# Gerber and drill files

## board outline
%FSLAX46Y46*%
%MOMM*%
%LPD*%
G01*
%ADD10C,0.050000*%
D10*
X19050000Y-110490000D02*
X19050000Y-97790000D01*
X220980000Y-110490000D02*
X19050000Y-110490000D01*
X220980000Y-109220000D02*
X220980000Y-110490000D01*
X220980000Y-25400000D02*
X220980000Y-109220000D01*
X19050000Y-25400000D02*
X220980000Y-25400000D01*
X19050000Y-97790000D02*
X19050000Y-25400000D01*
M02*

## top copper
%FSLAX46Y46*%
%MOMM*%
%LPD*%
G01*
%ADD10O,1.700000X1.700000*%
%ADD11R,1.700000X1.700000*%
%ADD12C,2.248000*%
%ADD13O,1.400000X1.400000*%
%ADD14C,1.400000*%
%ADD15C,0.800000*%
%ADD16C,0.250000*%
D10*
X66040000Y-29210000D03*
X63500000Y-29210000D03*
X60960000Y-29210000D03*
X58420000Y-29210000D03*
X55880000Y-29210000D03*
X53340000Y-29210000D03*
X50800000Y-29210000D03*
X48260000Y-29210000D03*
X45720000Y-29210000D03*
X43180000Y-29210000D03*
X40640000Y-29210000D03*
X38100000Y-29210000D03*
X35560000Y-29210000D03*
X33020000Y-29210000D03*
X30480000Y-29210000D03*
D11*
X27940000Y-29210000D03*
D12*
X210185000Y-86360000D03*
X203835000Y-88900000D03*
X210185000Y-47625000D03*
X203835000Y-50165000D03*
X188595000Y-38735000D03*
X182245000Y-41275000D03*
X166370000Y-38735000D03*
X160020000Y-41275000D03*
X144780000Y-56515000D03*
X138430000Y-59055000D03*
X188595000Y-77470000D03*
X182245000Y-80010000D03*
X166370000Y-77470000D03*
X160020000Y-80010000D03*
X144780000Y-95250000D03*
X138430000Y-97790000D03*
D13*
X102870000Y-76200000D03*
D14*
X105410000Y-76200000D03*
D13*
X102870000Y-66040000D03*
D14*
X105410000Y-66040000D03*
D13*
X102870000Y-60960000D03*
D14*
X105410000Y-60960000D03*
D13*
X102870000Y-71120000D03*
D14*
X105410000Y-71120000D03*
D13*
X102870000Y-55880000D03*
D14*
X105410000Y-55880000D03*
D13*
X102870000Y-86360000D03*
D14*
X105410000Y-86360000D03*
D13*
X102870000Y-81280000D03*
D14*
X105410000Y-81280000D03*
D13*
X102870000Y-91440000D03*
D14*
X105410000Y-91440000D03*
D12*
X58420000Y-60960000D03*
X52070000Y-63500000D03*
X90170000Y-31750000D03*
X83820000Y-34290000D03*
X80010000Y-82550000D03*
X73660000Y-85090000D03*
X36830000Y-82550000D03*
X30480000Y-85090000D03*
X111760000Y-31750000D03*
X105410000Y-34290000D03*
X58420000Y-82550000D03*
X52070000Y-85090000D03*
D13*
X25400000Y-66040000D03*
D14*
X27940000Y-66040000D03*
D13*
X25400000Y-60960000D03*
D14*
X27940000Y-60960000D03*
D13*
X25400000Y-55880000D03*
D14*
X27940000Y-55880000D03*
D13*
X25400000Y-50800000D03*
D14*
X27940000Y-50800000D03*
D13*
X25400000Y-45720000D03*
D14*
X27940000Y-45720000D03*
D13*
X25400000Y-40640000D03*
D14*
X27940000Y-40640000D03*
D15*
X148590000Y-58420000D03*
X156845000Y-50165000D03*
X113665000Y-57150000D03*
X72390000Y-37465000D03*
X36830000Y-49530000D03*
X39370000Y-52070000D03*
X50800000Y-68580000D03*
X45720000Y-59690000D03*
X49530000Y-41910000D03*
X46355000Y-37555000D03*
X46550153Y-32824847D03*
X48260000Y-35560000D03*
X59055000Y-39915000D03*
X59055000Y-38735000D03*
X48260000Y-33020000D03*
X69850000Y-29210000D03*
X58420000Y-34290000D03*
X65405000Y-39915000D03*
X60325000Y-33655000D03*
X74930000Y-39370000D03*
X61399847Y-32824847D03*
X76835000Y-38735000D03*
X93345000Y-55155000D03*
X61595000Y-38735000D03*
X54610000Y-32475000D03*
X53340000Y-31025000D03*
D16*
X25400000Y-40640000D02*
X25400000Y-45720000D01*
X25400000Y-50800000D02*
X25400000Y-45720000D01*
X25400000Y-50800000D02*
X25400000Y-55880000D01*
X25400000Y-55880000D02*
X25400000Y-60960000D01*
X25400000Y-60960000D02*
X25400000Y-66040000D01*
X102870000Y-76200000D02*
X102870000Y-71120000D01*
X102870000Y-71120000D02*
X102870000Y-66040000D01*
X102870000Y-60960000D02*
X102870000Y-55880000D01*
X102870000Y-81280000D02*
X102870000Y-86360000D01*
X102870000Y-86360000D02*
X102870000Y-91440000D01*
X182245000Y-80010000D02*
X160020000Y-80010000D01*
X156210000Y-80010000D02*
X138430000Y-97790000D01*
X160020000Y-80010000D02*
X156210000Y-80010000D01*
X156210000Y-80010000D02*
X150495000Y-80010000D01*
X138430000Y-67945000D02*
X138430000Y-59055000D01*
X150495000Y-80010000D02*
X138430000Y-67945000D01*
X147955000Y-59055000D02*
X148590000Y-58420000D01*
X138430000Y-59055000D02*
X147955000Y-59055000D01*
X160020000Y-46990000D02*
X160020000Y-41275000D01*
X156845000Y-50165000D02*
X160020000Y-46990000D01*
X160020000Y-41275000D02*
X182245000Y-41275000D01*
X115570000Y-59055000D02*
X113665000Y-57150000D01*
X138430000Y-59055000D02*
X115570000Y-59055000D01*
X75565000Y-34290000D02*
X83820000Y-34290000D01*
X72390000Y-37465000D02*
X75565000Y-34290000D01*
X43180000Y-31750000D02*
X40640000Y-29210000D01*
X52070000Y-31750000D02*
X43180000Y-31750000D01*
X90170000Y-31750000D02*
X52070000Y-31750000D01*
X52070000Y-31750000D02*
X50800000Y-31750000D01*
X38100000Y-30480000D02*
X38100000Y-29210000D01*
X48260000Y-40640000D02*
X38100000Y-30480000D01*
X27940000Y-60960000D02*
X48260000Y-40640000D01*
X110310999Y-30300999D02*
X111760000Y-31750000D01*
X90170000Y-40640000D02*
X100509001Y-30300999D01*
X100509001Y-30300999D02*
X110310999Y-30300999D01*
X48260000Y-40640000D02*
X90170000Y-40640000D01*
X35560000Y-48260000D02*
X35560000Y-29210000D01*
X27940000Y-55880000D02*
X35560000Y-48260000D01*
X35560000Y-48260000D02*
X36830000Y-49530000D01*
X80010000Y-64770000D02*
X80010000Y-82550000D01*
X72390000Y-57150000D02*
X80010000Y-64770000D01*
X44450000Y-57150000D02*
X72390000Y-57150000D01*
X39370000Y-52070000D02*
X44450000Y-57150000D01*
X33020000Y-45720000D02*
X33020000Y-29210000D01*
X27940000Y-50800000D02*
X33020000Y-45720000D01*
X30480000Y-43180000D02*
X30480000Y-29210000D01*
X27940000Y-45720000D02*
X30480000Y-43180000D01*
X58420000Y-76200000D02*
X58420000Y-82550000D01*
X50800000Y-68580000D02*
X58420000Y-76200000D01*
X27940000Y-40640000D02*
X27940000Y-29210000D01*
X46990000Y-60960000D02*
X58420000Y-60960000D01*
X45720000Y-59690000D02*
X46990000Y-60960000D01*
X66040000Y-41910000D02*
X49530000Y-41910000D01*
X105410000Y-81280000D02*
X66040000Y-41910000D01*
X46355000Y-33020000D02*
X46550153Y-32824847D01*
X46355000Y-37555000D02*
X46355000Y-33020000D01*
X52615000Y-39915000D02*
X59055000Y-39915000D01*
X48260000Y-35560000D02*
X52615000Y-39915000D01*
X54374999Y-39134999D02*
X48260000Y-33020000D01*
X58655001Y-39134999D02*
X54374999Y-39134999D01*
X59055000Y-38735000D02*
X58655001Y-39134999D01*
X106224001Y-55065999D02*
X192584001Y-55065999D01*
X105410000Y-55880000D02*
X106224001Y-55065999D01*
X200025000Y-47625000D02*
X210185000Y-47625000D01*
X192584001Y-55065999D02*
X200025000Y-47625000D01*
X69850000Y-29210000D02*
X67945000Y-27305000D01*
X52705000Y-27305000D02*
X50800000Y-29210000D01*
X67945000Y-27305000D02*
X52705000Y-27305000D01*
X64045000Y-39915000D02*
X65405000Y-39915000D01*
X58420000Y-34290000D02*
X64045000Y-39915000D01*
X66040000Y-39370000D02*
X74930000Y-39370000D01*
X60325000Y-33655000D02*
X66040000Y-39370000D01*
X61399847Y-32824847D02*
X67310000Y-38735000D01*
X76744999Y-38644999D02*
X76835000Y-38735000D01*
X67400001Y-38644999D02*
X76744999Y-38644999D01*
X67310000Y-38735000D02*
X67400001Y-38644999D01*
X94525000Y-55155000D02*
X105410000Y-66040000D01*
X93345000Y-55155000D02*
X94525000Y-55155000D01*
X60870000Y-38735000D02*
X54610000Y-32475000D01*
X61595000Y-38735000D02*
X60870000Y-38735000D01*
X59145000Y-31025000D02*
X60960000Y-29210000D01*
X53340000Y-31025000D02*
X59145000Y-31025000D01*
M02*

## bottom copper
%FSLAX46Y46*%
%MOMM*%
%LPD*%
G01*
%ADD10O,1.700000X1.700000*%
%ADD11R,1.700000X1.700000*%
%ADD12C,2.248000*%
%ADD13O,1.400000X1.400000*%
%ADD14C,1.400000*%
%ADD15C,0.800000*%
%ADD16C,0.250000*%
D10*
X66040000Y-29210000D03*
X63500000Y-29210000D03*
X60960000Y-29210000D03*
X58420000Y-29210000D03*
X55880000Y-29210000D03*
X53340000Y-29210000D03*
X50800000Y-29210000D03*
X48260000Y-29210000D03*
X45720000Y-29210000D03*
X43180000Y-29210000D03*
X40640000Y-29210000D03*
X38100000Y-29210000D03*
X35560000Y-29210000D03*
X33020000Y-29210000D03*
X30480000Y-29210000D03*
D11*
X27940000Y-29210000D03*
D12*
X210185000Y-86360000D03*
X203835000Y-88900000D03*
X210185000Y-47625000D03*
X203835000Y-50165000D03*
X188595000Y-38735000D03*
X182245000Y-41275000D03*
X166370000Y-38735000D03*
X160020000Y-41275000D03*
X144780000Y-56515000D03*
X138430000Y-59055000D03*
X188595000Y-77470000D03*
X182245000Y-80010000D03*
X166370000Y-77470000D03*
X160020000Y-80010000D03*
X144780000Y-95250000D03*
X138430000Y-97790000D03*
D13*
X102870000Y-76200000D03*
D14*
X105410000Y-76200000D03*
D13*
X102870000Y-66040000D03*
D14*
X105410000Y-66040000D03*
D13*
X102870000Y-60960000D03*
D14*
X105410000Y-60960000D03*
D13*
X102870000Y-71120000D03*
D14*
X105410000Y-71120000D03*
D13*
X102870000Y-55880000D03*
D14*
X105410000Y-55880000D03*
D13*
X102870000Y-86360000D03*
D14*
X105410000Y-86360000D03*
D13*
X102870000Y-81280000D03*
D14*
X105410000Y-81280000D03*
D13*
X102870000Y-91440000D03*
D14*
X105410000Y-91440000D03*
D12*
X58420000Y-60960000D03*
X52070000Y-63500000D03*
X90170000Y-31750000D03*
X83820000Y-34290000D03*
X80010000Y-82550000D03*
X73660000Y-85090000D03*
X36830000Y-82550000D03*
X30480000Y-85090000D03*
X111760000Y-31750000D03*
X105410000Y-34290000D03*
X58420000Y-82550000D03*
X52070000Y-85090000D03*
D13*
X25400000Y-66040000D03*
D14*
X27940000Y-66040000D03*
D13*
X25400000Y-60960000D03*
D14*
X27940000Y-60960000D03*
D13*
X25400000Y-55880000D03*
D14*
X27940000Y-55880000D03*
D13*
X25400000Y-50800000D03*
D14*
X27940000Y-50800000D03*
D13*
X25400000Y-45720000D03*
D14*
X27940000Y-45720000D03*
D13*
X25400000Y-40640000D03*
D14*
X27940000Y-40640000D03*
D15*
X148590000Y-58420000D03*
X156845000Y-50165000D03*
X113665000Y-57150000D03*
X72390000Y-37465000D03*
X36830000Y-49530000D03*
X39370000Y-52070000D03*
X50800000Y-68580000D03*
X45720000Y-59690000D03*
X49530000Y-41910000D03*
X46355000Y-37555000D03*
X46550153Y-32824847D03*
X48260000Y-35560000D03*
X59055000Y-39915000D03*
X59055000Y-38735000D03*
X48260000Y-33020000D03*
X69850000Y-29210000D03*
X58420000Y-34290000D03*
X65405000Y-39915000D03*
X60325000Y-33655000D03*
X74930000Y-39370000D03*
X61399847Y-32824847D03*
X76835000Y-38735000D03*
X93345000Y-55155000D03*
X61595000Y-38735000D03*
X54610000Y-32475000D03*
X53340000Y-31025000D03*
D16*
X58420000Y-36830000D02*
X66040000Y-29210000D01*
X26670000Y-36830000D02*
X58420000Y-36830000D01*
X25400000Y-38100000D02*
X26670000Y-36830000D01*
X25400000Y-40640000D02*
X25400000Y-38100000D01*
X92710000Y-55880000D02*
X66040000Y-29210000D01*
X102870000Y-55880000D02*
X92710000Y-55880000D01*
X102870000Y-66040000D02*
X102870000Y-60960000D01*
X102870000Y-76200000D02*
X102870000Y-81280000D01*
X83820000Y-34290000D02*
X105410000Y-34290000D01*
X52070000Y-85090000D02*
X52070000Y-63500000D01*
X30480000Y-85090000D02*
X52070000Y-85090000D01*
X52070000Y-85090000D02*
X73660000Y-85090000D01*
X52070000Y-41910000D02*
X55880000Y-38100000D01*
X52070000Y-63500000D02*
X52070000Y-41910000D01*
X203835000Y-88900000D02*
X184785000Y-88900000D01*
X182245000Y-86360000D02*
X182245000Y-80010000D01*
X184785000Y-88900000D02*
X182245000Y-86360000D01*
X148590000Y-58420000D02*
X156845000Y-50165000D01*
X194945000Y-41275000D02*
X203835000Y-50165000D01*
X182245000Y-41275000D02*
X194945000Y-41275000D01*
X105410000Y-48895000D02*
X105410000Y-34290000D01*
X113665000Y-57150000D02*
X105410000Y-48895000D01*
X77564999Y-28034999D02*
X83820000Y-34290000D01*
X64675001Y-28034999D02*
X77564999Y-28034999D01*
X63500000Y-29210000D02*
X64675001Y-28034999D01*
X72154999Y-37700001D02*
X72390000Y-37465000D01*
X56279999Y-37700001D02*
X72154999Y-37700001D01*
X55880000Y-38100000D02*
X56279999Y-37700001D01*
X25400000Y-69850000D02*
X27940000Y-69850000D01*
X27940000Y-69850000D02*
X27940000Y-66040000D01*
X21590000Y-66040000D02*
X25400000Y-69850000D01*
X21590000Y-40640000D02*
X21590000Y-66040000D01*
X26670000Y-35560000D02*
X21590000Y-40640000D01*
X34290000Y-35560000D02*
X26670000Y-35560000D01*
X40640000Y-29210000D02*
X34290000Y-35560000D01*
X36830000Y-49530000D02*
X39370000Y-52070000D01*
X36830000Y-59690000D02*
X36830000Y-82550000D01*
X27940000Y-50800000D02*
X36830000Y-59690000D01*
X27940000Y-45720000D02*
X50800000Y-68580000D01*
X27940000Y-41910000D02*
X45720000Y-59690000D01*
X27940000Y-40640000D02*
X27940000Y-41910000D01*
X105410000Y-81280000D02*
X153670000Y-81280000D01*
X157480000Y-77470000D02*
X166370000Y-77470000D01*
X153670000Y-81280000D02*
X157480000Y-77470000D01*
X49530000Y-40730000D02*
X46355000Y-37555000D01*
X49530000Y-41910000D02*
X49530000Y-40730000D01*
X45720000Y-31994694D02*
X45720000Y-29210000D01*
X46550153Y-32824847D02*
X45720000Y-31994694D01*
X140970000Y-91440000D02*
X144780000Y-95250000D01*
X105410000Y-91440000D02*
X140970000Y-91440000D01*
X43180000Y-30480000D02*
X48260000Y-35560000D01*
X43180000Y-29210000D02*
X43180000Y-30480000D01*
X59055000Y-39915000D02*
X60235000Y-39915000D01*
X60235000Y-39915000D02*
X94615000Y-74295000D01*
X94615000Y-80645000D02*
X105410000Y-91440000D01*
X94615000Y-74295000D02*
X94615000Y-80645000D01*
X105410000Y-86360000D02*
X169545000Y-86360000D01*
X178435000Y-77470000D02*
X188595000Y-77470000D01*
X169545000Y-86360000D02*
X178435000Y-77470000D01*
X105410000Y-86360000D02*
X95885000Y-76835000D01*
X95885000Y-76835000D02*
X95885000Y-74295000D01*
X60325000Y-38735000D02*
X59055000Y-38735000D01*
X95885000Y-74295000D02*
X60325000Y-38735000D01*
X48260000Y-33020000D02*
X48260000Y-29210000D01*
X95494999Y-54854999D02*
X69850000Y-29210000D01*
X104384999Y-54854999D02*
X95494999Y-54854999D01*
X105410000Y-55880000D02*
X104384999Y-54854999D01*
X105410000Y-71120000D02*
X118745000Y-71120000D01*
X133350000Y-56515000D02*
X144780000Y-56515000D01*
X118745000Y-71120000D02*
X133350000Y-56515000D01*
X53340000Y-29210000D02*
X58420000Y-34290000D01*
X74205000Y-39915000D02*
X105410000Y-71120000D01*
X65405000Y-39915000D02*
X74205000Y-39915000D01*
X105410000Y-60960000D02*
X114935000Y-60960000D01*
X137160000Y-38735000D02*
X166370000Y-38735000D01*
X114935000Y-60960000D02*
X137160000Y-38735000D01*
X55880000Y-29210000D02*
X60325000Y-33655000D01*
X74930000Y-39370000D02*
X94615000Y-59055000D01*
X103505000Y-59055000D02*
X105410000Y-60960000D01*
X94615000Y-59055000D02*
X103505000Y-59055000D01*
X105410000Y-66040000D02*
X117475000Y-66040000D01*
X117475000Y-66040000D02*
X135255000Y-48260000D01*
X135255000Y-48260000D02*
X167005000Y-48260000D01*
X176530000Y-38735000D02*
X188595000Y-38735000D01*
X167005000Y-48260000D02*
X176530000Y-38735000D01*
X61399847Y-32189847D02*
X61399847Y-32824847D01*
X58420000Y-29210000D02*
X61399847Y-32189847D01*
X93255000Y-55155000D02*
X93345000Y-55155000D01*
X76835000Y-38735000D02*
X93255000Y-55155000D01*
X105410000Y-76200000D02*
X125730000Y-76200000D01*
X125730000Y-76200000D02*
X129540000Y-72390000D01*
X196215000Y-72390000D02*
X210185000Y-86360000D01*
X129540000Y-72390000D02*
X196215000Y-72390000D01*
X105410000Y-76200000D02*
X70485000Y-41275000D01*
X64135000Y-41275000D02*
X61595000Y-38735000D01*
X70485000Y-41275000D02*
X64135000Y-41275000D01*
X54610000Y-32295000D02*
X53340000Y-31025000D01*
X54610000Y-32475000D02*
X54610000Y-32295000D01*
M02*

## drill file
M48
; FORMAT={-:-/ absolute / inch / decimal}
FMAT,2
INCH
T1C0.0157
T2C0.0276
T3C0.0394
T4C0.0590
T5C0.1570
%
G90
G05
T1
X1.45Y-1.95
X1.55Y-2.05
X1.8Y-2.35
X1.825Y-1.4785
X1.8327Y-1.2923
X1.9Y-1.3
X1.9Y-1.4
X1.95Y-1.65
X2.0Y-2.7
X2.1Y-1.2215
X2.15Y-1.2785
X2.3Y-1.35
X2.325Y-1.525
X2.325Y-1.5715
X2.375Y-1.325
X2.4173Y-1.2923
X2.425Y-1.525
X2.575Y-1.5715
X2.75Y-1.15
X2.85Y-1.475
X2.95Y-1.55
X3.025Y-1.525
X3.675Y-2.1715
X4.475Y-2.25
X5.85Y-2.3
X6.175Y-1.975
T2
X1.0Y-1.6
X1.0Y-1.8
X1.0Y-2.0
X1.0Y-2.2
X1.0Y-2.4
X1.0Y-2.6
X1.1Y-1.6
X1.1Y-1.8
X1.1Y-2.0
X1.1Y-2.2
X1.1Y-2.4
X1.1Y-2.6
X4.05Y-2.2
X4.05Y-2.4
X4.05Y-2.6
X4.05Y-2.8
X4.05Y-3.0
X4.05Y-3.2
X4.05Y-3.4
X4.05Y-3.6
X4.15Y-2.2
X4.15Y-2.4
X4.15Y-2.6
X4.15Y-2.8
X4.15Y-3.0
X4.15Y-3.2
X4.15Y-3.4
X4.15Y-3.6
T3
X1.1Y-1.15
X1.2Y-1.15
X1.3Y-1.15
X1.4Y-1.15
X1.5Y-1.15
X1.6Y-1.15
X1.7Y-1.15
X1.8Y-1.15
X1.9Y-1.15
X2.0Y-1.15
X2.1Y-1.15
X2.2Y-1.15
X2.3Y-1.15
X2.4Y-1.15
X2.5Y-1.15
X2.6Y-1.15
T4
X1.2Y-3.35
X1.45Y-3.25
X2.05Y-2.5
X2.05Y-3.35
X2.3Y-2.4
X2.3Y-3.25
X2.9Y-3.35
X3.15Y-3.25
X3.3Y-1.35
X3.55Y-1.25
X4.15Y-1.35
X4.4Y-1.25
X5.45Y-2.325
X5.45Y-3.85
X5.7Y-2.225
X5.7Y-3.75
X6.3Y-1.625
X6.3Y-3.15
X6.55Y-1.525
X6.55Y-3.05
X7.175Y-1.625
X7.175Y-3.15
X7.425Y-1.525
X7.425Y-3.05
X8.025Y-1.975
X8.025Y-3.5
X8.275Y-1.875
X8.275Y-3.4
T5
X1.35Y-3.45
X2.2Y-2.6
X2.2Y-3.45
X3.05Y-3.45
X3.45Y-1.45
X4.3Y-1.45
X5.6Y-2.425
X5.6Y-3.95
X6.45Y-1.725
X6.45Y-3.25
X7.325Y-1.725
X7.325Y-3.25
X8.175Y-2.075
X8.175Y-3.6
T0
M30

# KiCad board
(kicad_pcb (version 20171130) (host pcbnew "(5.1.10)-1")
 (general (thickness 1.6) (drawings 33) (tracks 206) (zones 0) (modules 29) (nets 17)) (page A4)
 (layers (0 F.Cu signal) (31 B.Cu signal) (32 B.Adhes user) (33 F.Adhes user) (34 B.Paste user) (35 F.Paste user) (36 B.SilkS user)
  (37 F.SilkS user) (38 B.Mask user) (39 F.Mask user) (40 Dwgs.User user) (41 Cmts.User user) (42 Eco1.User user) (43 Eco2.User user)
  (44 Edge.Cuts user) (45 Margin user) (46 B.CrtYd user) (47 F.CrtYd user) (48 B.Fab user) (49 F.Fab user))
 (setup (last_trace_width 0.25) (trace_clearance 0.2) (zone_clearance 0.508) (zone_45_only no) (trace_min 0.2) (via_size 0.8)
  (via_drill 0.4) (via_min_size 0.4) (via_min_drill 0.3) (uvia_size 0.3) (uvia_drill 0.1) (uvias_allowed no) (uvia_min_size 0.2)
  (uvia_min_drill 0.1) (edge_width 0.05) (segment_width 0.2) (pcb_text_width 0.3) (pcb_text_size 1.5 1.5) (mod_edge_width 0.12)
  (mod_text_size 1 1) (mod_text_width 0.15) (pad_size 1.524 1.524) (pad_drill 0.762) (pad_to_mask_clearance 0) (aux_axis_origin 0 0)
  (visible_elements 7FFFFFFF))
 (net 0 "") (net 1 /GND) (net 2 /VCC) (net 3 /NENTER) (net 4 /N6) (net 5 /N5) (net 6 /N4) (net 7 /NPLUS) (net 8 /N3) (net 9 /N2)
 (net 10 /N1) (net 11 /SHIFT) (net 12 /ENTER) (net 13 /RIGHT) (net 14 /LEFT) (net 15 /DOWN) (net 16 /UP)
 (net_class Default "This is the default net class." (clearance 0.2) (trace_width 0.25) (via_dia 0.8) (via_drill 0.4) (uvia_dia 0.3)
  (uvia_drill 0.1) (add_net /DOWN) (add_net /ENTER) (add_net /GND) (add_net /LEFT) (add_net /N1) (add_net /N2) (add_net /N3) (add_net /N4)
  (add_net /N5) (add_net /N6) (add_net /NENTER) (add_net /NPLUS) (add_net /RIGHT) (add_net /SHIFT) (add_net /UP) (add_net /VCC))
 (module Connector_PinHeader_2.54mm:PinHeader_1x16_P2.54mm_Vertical (layer F.Cu) (at 27.94 29.21 90)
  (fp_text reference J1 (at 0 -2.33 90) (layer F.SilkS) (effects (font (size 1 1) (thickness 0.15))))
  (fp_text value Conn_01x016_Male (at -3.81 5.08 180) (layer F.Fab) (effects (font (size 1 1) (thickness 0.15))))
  (pad 16 thru_hole oval (at 0 38.1 90) (size 1.7 1.7) (drill 1) (layers *.Cu *.Mask) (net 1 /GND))
  (pad 15 thru_hole oval (at 0 35.56 90) (size 1.7 1.7) (drill 1) (layers *.Cu *.Mask) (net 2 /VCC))
  (pad 14 thru_hole oval (at 0 33.02 90) (size 1.7 1.7) (drill 1) (layers *.Cu *.Mask) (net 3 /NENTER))
  (pad 13 thru_hole oval (at 0 30.48 90) (size 1.7 1.7) (drill 1) (layers *.Cu *.Mask) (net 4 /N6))
  (pad 12 thru_hole oval (at 0 27.94 90) (size 1.7 1.7) (drill 1) (layers *.Cu *.Mask) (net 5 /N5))
  (pad 11 thru_hole oval (at 0 25.4 90) (size 1.7 1.7) (drill 1) (layers *.Cu *.Mask) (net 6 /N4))
  (pad 10 thru_hole oval (at 0 22.86 90) (size 1.7 1.7) (drill 1) (layers *.Cu *.Mask) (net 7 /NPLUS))
  (pad 9 thru_hole oval (at 0 20.32 90) (size 1.7 1.7) (drill 1) (layers *.Cu *.Mask) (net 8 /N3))
  (pad 8 thru_hole oval (at 0 17.78 90) (size 1.7 1.7) (drill 1) (layers *.Cu *.Mask) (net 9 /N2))
  (pad 7 thru_hole oval (at 0 15.24 90) (size 1.7 1.7) (drill 1) (layers *.Cu *.Mask) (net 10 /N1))
  (pad 6 thru_hole oval (at 0 12.7 90) (size 1.7 1.7) (drill 1) (layers *.Cu *.Mask) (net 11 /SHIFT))
  (pad 5 thru_hole oval (at 0 10.16 90) (size 1.7 1.7) (drill 1) (layers *.Cu *.Mask) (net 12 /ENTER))
  (pad 4 thru_hole oval (at 0 7.62 90) (size 1.7 1.7) (drill 1) (layers *.Cu *.Mask) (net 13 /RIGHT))
  (pad 3 thru_hole oval (at 0 5.08 90) (size 1.7 1.7) (drill 1) (layers *.Cu *.Mask) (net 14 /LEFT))
  (pad 2 thru_hole oval (at 0 2.54 90) (size 1.7 1.7) (drill 1) (layers *.Cu *.Mask) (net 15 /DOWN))
  (pad 1 thru_hole rect (at 0 0 90) (size 1.7 1.7) (drill 1) (layers *.Cu *.Mask) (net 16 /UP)))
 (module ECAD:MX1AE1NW (layer F.Cu) (at 203.835 88.9)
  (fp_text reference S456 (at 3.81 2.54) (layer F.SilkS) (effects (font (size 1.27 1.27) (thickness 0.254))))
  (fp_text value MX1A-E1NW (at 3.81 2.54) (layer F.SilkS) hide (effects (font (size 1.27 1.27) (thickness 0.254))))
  (pad MH1 np_thru_hole circle (at 3.81 2.54) (size 3.9878 0) (drill 3.9878) (layers *.Cu *.Mask))
  (pad 2 thru_hole circle (at 6.35 -2.54) (size 2.248 2.248) (drill 1.4986) (layers *.Cu *.Mask) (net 3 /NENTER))
  (pad 1 thru_hole circle (at 0 0) (size 2.248 2.248) (drill 1.4986) (layers *.Cu *.Mask) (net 2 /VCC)))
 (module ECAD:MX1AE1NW (layer F.Cu) (at 203.835 50.165)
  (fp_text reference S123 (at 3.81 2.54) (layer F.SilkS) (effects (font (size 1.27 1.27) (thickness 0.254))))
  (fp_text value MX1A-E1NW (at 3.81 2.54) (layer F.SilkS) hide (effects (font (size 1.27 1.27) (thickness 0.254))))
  (pad MH1 np_thru_hole circle (at 3.81 2.54) (size 3.9878 0) (drill 3.9878) (layers *.Cu *.Mask))
  (pad 2 thru_hole circle (at 6.35 -2.54) (size 2.248 2.248) (drill 1.4986) (layers *.Cu *.Mask) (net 7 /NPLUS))
  (pad 1 thru_hole circle (at 0 0) (size 2.248 2.248) (drill 1.4986) (layers *.Cu *.Mask) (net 2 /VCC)))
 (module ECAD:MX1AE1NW (layer F.Cu) (at 182.245 41.275)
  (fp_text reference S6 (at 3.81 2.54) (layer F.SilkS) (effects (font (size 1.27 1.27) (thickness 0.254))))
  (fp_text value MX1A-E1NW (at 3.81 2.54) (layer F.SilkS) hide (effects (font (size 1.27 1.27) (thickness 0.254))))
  (pad MH1 np_thru_hole circle (at 3.81 2.54) (size 3.9878 0) (drill 3.9878) (layers *.Cu *.Mask))
  (pad 2 thru_hole circle (at 6.35 -2.54) (size 2.248 2.248) (drill 1.4986) (layers *.Cu *.Mask) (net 4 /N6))
  (pad 1 thru_hole circle (at 0 0) (size 2.248 2.248) (drill 1.4986) (layers *.Cu *.Mask) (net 2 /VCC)))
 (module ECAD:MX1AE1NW (layer F.Cu) (at 160.02 41.275)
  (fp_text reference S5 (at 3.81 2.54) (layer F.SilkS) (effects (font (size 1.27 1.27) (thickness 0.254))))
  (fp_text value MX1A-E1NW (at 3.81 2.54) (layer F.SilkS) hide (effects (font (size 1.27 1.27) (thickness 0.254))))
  (pad MH1 np_thru_hole circle (at 3.81 2.54) (size 3.9878 0) (drill 3.9878) (layers *.Cu *.Mask))
  (pad 2 thru_hole circle (at 6.35 -2.54) (size 2.248 2.248) (drill 1.4986) (layers *.Cu *.Mask) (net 5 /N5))
  (pad 1 thru_hole circle (at 0 0) (size 2.248 2.248) (drill 1.4986) (layers *.Cu *.Mask) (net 2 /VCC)))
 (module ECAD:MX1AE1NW (layer F.Cu) (at 138.43 59.055)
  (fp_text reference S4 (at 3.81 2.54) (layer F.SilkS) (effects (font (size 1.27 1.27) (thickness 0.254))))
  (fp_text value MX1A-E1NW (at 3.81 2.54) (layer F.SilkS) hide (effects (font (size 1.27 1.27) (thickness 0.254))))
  (pad MH1 np_thru_hole circle (at 3.81 2.54) (size 3.9878 0) (drill 3.9878) (layers *.Cu *.Mask))
  (pad 2 thru_hole circle (at 6.35 -2.54) (size 2.248 2.248) (drill 1.4986) (layers *.Cu *.Mask) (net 6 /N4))
  (pad 1 thru_hole circle (at 0 0) (size 2.248 2.248) (drill 1.4986) (layers *.Cu *.Mask) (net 2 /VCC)))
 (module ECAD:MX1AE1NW (layer F.Cu) (at 182.245 80.01)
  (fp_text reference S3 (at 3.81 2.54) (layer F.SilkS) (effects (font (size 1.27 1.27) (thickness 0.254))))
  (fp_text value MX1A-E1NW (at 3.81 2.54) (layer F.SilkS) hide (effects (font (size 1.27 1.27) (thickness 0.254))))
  (pad MH1 np_thru_hole circle (at 3.81 2.54) (size 3.9878 0) (drill 3.9878) (layers *.Cu *.Mask))
  (pad 2 thru_hole circle (at 6.35 -2.54) (size 2.248 2.248) (drill 1.4986) (layers *.Cu *.Mask) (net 8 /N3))
  (pad 1 thru_hole circle (at 0 0) (size 2.248 2.248) (drill 1.4986) (layers *.Cu *.Mask) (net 2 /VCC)))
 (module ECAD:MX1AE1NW (layer F.Cu) (at 160.02 80.01)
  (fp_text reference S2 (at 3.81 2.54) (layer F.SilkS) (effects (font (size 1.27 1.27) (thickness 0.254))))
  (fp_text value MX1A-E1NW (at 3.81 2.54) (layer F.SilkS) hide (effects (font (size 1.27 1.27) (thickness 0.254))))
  (pad MH1 np_thru_hole circle (at 3.81 2.54) (size 3.9878 0) (drill 3.9878) (layers *.Cu *.Mask))
  (pad 2 thru_hole circle (at 6.35 -2.54) (size 2.248 2.248) (drill 1.4986) (layers *.Cu *.Mask) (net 9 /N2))
  (pad 1 thru_hole circle (at 0 0) (size 2.248 2.248) (drill 1.4986) (layers *.Cu *.Mask) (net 2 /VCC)))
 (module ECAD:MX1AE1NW (layer F.Cu) (at 138.43 97.79)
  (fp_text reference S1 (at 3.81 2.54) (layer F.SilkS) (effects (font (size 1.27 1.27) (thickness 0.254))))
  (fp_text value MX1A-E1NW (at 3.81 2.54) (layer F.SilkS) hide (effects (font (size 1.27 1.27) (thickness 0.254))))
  (pad MH1 np_thru_hole circle (at 3.81 2.54) (size 3.9878 0) (drill 3.9878) (layers *.Cu *.Mask))
  (pad 2 thru_hole circle (at 6.35 -2.54) (size 2.248 2.248) (drill 1.4986) (layers *.Cu *.Mask) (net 10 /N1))
  (pad 1 thru_hole circle (at 0 0) (size 2.248 2.248) (drill 1.4986) (layers *.Cu *.Mask) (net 2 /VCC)))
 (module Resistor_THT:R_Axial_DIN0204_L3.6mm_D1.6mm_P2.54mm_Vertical (layer F.Cu) (at 105.41 76.2 180)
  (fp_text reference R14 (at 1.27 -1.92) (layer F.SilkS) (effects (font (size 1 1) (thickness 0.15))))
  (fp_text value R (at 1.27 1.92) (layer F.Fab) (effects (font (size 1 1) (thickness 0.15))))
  (pad 2 thru_hole oval (at 2.54 0 180) (size 1.4 1.4) (drill 0.7) (layers *.Cu *.Mask) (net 1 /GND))
  (pad 1 thru_hole circle (at 0 0 180) (size 1.4 1.4) (drill 0.7) (layers *.Cu *.Mask) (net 3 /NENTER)))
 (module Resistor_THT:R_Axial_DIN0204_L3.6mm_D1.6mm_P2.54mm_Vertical (layer F.Cu) (at 105.41 66.04 180)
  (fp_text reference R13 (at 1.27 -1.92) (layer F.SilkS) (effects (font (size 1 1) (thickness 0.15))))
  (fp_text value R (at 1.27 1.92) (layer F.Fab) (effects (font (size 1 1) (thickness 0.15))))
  (pad 2 thru_hole oval (at 2.54 0 180) (size 1.4 1.4) (drill 0.7) (layers *.Cu *.Mask) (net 1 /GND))
  (pad 1 thru_hole circle (at 0 0 180) (size 1.4 1.4) (drill 0.7) (layers *.Cu *.Mask) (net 4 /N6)))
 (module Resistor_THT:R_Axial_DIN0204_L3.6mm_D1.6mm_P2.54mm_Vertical (layer F.Cu) (at 105.41 60.96 180)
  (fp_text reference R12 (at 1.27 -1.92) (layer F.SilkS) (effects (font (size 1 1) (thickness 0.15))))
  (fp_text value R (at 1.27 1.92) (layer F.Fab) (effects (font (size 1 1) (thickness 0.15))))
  (pad 2 thru_hole oval (at 2.54 0 180) (size 1.4 1.4) (drill 0.7) (layers *.Cu *.Mask) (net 1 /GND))
  (pad 1 thru_hole circle (at 0 0 180) (size 1.4 1.4) (drill 0.7) (layers *.Cu *.Mask) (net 5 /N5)))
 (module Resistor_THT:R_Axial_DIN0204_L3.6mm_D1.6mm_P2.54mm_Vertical (layer F.Cu) (at 105.41 71.12 180)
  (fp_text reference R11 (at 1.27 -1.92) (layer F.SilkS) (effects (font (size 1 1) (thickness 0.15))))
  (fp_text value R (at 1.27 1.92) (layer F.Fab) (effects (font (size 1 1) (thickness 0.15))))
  (pad 2 thru_hole oval (at 2.54 0 180) (size 1.4 1.4) (drill 0.7) (layers *.Cu *.Mask) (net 1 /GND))
  (pad 1 thru_hole circle (at 0 0 180) (size 1.4 1.4) (drill 0.7) (layers *.Cu *.Mask) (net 6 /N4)))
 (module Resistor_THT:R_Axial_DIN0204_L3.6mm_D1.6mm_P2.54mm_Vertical (layer F.Cu) (at 105.41 55.88 180)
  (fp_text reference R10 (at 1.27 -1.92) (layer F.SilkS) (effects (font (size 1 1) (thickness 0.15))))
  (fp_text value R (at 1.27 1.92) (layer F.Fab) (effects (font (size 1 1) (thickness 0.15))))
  (pad 2 thru_hole oval (at 2.54 0 180) (size 1.4 1.4) (drill 0.7) (layers *.Cu *.Mask) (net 1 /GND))
  (pad 1 thru_hole circle (at 0 0 180) (size 1.4 1.4) (drill 0.7) (layers *.Cu *.Mask) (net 7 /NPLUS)))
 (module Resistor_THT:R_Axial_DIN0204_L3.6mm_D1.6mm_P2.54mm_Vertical (layer F.Cu) (at 105.41 86.36 180)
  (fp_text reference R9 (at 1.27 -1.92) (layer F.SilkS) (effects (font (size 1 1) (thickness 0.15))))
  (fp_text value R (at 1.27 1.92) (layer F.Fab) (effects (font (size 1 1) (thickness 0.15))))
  (pad 2 thru_hole oval (at 2.54 0 180) (size 1.4 1.4) (drill 0.7) (layers *.Cu *.Mask) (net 1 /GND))
  (pad 1 thru_hole circle (at 0 0 180) (size 1.4 1.4) (drill 0.7) (layers *.Cu *.Mask) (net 8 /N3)))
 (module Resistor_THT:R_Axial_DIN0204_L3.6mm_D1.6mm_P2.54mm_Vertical (layer F.Cu) (at 105.41 81.28 180)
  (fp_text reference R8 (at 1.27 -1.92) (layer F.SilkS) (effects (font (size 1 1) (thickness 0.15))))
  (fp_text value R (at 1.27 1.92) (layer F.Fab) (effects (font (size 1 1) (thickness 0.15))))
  (pad 2 thru_hole oval (at 2.54 0 180) (size 1.4 1.4) (drill 0.7) (layers *.Cu *.Mask) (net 1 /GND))
  (pad 1 thru_hole circle (at 0 0 180) (size 1.4 1.4) (drill 0.7) (layers *.Cu *.Mask) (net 9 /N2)))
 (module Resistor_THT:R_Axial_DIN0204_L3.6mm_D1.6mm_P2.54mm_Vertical (layer F.Cu) (at 105.41 91.44 180)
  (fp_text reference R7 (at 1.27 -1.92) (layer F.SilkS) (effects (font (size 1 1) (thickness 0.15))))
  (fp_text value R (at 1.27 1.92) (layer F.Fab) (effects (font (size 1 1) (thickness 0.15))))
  (pad 2 thru_hole oval (at 2.54 0 180) (size 1.4 1.4) (drill 0.7) (layers *.Cu *.Mask) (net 1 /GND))
  (pad 1 thru_hole circle (at 0 0 180) (size 1.4 1.4) (drill 0.7) (layers *.Cu *.Mask) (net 10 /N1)))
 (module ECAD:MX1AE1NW (layer F.Cu) (at 52.07 63.5)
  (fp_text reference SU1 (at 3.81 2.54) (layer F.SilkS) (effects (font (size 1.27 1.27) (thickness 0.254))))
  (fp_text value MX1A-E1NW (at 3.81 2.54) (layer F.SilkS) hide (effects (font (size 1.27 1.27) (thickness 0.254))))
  (pad MH1 np_thru_hole circle (at 3.81 2.54) (size 3.9878 0) (drill 3.9878) (layers *.Cu *.Mask))
  (pad 2 thru_hole circle (at 6.35 -2.54) (size 2.248 2.248) (drill 1.4986) (layers *.Cu *.Mask) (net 16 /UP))
  (pad 1 thru_hole circle (at 0 0) (size 2.248 2.248) (drill 1.4986) (layers *.Cu *.Mask) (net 2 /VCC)))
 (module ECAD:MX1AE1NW (layer F.Cu) (at 83.82 34.29)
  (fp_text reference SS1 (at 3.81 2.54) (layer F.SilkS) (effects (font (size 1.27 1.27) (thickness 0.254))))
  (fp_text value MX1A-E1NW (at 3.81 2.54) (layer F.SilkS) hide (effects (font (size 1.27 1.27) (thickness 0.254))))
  (pad MH1 np_thru_hole circle (at 3.81 2.54) (size 3.9878 0) (drill 3.9878) (layers *.Cu *.Mask))
  (pad 2 thru_hole circle (at 6.35 -2.54) (size 2.248 2.248) (drill 1.4986) (layers *.Cu *.Mask) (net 11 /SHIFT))
  (pad 1 thru_hole circle (at 0 0) (size 2.248 2.248) (drill 1.4986) (layers *.Cu *.Mask) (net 2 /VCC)))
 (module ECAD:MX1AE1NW (layer F.Cu) (at 73.66 85.09)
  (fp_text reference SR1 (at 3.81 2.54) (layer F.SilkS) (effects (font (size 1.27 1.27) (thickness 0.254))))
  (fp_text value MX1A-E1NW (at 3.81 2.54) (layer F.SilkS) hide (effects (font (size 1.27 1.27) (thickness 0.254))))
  (pad MH1 np_thru_hole circle (at 3.81 2.54) (size 3.9878 0) (drill 3.9878) (layers *.Cu *.Mask))
  (pad 2 thru_hole circle (at 6.35 -2.54) (size 2.248 2.248) (drill 1.4986) (layers *.Cu *.Mask) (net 13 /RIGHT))
  (pad 1 thru_hole circle (at 0 0) (size 2.248 2.248) (drill 1.4986) (layers *.Cu *.Mask) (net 2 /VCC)))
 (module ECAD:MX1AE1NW (layer F.Cu) (at 30.48 85.09)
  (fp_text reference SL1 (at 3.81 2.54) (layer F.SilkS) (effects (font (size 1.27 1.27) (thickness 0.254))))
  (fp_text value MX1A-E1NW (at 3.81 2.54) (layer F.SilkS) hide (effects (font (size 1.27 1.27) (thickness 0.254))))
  (pad MH1 np_thru_hole circle (at 3.81 2.54) (size 3.9878 0) (drill 3.9878) (layers *.Cu *.Mask))
  (pad 2 thru_hole circle (at 6.35 -2.54) (size 2.248 2.248) (drill 1.4986) (layers *.Cu *.Mask) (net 14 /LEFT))
  (pad 1 thru_hole circle (at 0 0) (size 2.248 2.248) (drill 1.4986) (layers *.Cu *.Mask) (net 2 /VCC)))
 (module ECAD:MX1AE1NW (layer F.Cu) (at 105.41 34.29)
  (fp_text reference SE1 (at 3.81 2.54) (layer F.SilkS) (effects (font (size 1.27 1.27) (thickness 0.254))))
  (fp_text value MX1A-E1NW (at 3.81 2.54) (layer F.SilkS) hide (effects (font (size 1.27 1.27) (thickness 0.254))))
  (pad MH1 np_thru_hole circle (at 3.81 2.54) (size 3.9878 0) (drill 3.9878) (layers *.Cu *.Mask))
  (pad 2 thru_hole circle (at 6.35 -2.54) (size 2.248 2.248) (drill 1.4986) (layers *.Cu *.Mask) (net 12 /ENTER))
  (pad 1 thru_hole circle (at 0 0) (size 2.248 2.248) (drill 1.4986) (layers *.Cu *.Mask) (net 2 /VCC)))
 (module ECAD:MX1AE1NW (layer F.Cu) (at 52.07 85.09)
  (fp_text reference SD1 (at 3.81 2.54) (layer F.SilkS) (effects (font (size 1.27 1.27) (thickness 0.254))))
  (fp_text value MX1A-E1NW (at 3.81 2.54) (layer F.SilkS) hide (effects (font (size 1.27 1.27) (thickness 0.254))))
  (pad MH1 np_thru_hole circle (at 3.81 2.54) (size 3.9878 0) (drill 3.9878) (layers *.Cu *.Mask))
  (pad 2 thru_hole circle (at 6.35 -2.54) (size 2.248 2.248) (drill 1.4986) (layers *.Cu *.Mask) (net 15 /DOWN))
  (pad 1 thru_hole circle (at 0 0) (size 2.248 2.248) (drill 1.4986) (layers *.Cu *.Mask) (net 2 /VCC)))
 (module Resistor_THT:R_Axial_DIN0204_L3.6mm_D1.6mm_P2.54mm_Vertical (layer F.Cu) (at 27.94 66.04 180)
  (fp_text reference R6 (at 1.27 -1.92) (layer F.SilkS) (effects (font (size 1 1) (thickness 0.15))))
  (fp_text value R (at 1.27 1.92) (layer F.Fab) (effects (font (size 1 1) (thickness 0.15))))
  (pad 2 thru_hole oval (at 2.54 0 180) (size 1.4 1.4) (drill 0.7) (layers *.Cu *.Mask) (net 1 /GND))
  (pad 1 thru_hole circle (at 0 0 180) (size 1.4 1.4) (drill 0.7) (layers *.Cu *.Mask) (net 11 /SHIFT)))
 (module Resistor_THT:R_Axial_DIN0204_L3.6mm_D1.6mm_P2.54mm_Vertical (layer F.Cu) (at 27.94 60.96 180)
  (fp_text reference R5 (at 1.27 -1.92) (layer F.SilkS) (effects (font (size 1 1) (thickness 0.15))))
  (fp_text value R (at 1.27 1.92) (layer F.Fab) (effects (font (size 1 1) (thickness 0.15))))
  (pad 2 thru_hole oval (at 2.54 0 180) (size 1.4 1.4) (drill 0.7) (layers *.Cu *.Mask) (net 1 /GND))
  (pad 1 thru_hole circle (at 0 0 180) (size 1.4 1.4) (drill 0.7) (layers *.Cu *.Mask) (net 12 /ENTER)))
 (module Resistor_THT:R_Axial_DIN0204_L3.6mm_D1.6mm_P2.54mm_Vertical (layer F.Cu) (at 27.94 55.88 180)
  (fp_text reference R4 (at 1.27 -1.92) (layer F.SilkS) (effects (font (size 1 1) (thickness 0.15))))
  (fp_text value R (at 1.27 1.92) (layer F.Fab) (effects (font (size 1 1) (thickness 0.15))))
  (pad 2 thru_hole oval (at 2.54 0 180) (size 1.4 1.4) (drill 0.7) (layers *.Cu *.Mask) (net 1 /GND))
  (pad 1 thru_hole circle (at 0 0 180) (size 1.4 1.4) (drill 0.7) (layers *.Cu *.Mask) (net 13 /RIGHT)))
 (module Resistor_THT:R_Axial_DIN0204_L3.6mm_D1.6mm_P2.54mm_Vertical (layer F.Cu) (at 27.94 50.8 180)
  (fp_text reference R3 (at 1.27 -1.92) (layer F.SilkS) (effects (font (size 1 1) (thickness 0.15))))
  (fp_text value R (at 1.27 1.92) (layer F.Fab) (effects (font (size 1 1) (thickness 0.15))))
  (pad 2 thru_hole oval (at 2.54 0 180) (size 1.4 1.4) (drill 0.7) (layers *.Cu *.Mask) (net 1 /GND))
  (pad 1 thru_hole circle (at 0 0 180) (size 1.4 1.4) (drill 0.7) (layers *.Cu *.Mask) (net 14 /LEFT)))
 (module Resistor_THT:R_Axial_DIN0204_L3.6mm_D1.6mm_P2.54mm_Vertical (layer F.Cu) (at 27.94 45.72 180)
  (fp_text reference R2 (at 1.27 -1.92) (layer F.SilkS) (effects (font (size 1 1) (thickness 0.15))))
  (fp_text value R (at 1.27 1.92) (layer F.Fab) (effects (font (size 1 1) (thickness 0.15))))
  (pad 2 thru_hole oval (at 2.54 0 180) (size 1.4 1.4) (drill 0.7) (layers *.Cu *.Mask) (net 1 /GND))
  (pad 1 thru_hole circle (at 0 0 180) (size 1.4 1.4) (drill 0.7) (layers *.Cu *.Mask) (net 15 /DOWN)))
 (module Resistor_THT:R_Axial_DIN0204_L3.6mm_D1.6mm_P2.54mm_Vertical (layer F.Cu) (at 27.94 40.64 180)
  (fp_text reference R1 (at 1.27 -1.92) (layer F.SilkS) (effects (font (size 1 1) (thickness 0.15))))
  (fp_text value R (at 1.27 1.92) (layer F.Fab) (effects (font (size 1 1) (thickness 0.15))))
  (pad 2 thru_hole oval (at 2.54 0 180) (size 1.4 1.4) (drill 0.7) (layers *.Cu *.Mask) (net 1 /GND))
  (pad 1 thru_hole circle (at 0 0 180) (size 1.4 1.4) (drill 0.7) (layers *.Cu *.Mask) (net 16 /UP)))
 (gr_line (start 19.05 110.49) (end 19.05 97.79) (layer Edge.Cuts) (width 0.05))
 (gr_line (start 220.98 110.49) (end 19.05 110.49) (layer Edge.Cuts) (width 0.05))
 (gr_line (start 220.98 109.22) (end 220.98 110.49) (layer Edge.Cuts) (width 0.05))
 (gr_line (start 220.98 25.4) (end 220.98 109.22) (layer Edge.Cuts) (width 0.05))
 (gr_line (start 19.05 25.4) (end 220.98 25.4) (layer Edge.Cuts) (width 0.05))
 (gr_line (start 19.05 97.79) (end 19.05 25.4) (layer Edge.Cuts) (width 0.05))
 (segment (start 25.4 40.64) (end 25.4 45.72) (width 0.25) (layer F.Cu) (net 1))
 (segment (start 25.4 50.8) (end 25.4 45.72) (width 0.25) (layer F.Cu) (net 1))
 (segment (start 25.4 50.8) (end 25.4 55.88) (width 0.25) (layer F.Cu) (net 1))
 (segment (start 25.4 55.88) (end 25.4 60.96) (width 0.25) (layer F.Cu) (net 1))
 (segment (start 25.4 60.96) (end 25.4 66.04) (width 0.25) (layer F.Cu) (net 1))
 (segment (start 58.42 36.83) (end 66.04 29.21) (width 0.25) (layer B.Cu) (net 1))
 (segment (start 26.67 36.83) (end 58.42 36.83) (width 0.25) (layer B.Cu) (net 1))
 (segment (start 25.4 38.1) (end 26.67 36.83) (width 0.25) (layer B.Cu) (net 1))
 (segment (start 25.4 40.64) (end 25.4 38.1) (width 0.25) (layer B.Cu) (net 1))
 (segment (start 102.87 76.2) (end 102.87 71.12) (width 0.25) (layer F.Cu) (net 1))
 (segment (start 92.71 55.88) (end 66.04 29.21) (width 0.25) (layer B.Cu) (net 1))
 (segment (start 102.87 55.88) (end 92.71 55.88) (width 0.25) (layer B.Cu) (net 1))
 (segment (start 102.87 71.12) (end 102.87 66.04) (width 0.25) (layer F.Cu) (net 1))
 (segment (start 102.87 66.04) (end 102.87 60.96) (width 0.25) (layer B.Cu) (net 1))
 (segment (start 102.87 60.96) (end 102.87 55.88) (width 0.25) (layer F.Cu) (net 1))
 (segment (start 102.87 76.2) (end 102.87 81.28) (width 0.25) (layer B.Cu) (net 1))
 (segment (start 102.87 81.28) (end 102.87 86.36) (width 0.25) (layer F.Cu) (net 1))
 (segment (start 102.87 86.36) (end 102.87 91.44) (width 0.25) (layer F.Cu) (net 1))
 (segment (start 83.82 34.29) (end 105.41 34.29) (width 0.25) (layer B.Cu) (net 2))
 (segment (start 52.07 85.09) (end 52.07 63.5) (width 0.25) (layer B.Cu) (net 2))
 (segment (start 30.48 85.09) (end 52.07 85.09) (width 0.25) (layer B.Cu) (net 2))
 (segment (start 52.07 85.09) (end 73.66 85.09) (width 0.25) (layer B.Cu) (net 2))
 (segment (start 52.07 41.91) (end 55.88 38.1) (width 0.25) (layer B.Cu) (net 2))
 (segment (start 52.07 63.5) (end 52.07 41.91) (width 0.25) (layer B.Cu) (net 2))
 (segment (start 203.835 88.9) (end 184.785 88.9) (width 0.25) (layer B.Cu) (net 2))
 (segment (start 182.245 86.36) (end 182.245 80.01) (width 0.25) (layer B.Cu) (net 2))
 (segment (start 184.785 88.9) (end 182.245 86.36) (width 0.25) (layer B.Cu) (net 2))
 (segment (start 182.245 80.01) (end 160.02 80.01) (width 0.25) (layer F.Cu) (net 2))
 (segment (start 156.21 80.01) (end 138.43 97.79) (width 0.25) (layer F.Cu) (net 2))
 (segment (start 160.02 80.01) (end 156.21 80.01) (width 0.25) (layer F.Cu) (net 2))
 (segment (start 156.21 80.01) (end 150.495 80.01) (width 0.25) (layer F.Cu) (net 2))
 (segment (start 138.43 67.945) (end 138.43 59.055) (width 0.25) (layer F.Cu) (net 2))
 (segment (start 150.495 80.01) (end 138.43 67.945) (width 0.25) (layer F.Cu) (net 2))
 (via (at 148.59 58.42) (size 0.8) (drill 0.4) (layers F.Cu B.Cu) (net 2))
 (segment (start 147.955 59.055) (end 148.59 58.42) (width 0.25) (layer F.Cu) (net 2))
 (segment (start 138.43 59.055) (end 147.955 59.055) (width 0.25) (layer F.Cu) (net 2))
 (via (at 156.845 50.165) (size 0.8) (drill 0.4) (layers F.Cu B.Cu) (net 2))
 (segment (start 148.59 58.42) (end 156.845 50.165) (width 0.25) (layer B.Cu) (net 2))
 (segment (start 160.02 46.99) (end 160.02 41.275) (width 0.25) (layer F.Cu) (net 2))
 (segment (start 156.845 50.165) (end 160.02 46.99) (width 0.25) (layer F.Cu) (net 2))
 (segment (start 160.02 41.275) (end 182.245 41.275) (width 0.25) (layer F.Cu) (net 2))
 (segment (start 194.945 41.275) (end 203.835 50.165) (width 0.25) (layer B.Cu) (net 2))
 (segment (start 182.245 41.275) (end 194.945 41.275) (width 0.25) (layer B.Cu) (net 2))
 (via (at 113.665 57.15) (size 0.8) (drill 0.4) (layers F.Cu B.Cu) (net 2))
 (segment (start 115.57 59.055) (end 113.665 57.15) (width 0.25) (layer F.Cu) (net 2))
 (segment (start 138.43 59.055) (end 115.57 59.055) (width 0.25) (layer F.Cu) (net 2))
 (segment (start 105.41 48.895) (end 105.41 34.29) (width 0.25) (layer B.Cu) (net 2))
 (segment (start 113.665 57.15) (end 105.41 48.895) (width 0.25) (layer B.Cu) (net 2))
 (segment (start 77.564999 28.034999) (end 83.82 34.29) (width 0.25) (layer B.Cu) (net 2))
 (segment (start 64.675001 28.034999) (end 77.564999 28.034999) (width 0.25) (layer B.Cu) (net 2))
 (segment (start 63.5 29.21) (end 64.675001 28.034999) (width 0.25) (layer B.Cu) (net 2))
 (via (at 72.39 37.465) (size 0.8) (drill 0.4) (layers F.Cu B.Cu) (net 2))
 (segment (start 72.154999 37.700001) (end 72.39 37.465) (width 0.25) (layer B.Cu) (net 2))
 (segment (start 56.279999 37.700001) (end 72.154999 37.700001) (width 0.25) (layer B.Cu) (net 2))
 (segment (start 55.88 38.1) (end 56.279999 37.700001) (width 0.25) (layer B.Cu) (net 2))
 (segment (start 75.565 34.29) (end 83.82 34.29) (width 0.25) (layer F.Cu) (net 2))
 (segment (start 72.39 37.465) (end 75.565 34.29) (width 0.25) (layer F.Cu) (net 2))
 (segment (start 25.4 69.85) (end 27.94 69.85) (width 0.25) (layer B.Cu) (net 11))
 (segment (start 27.94 69.85) (end 27.94 66.04) (width 0.25) (layer B.Cu) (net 11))
 (segment (start 21.59 66.04) (end 25.4 69.85) (width 0.25) (layer B.Cu) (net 11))
 (segment (start 21.59 40.64) (end 21.59 66.04) (width 0.25) (layer B.Cu) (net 11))
 (segment (start 26.67 35.56) (end 21.59 40.64) (width 0.25) (layer B.Cu) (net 11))
 (segment (start 34.29 35.56) (end 26.67 35.56) (width 0.25) (layer B.Cu) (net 11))
 (segment (start 40.64 29.21) (end 34.29 35.56) (width 0.25) (layer B.Cu) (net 11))
 (segment (start 43.18 31.75) (end 40.64 29.21) (width 0.25) (layer F.Cu) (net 11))
 (segment (start 52.07 31.75) (end 43.18 31.75) (width 0.25) (layer F.Cu) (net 11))
 (segment (start 90.17 31.75) (end 52.07 31.75) (width 0.25) (layer F.Cu) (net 11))
 (segment (start 52.07 31.75) (end 50.8 31.75) (width 0.25) (layer F.Cu) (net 11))
 (segment (start 38.1 30.48) (end 38.1 29.21) (width 0.25) (layer F.Cu) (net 12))
 (segment (start 48.26 40.64) (end 38.1 30.48) (width 0.25) (layer F.Cu) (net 12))
 (segment (start 27.94 60.96) (end 48.26 40.64) (width 0.25) (layer F.Cu) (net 12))
 (segment (start 110.310999 30.300999) (end 111.76 31.75) (width 0.25) (layer F.Cu) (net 12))
 (segment (start 90.17 40.64) (end 100.509001 30.300999) (width 0.25) (layer F.Cu) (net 12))
 (segment (start 100.509001 30.300999) (end 110.310999 30.300999) (width 0.25) (layer F.Cu) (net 12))
 (segment (start 48.26 40.64) (end 90.17 40.64) (width 0.25) (layer F.Cu) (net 12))
 (segment (start 35.56 48.26) (end 35.56 29.21) (width 0.25) (layer F.Cu) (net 13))
 (segment (start 27.94 55.88) (end 35.56 48.26) (width 0.25) (layer F.Cu) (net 13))
 (via (at 36.83 49.53) (size 0.8) (drill 0.4) (layers F.Cu B.Cu) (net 13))
 (segment (start 35.56 48.26) (end 36.83 49.53) (width 0.25) (layer F.Cu) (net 13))
 (via (at 39.37 52.07) (size 0.8) (drill 0.4) (layers F.Cu B.Cu) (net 13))
 (segment (start 36.83 49.53) (end 39.37 52.07) (width 0.25) (layer B.Cu) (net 13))
 (segment (start 80.01 64.77) (end 80.01 82.55) (width 0.25) (layer F.Cu) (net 13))
 (segment (start 72.39 57.15) (end 80.01 64.77) (width 0.25) (layer F.Cu) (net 13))
 (segment (start 44.45 57.15) (end 72.39 57.15) (width 0.25) (layer F.Cu) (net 13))
 (segment (start 39.37 52.07) (end 44.45 57.15) (width 0.25) (layer F.Cu) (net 13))
 (segment (start 33.02 45.72) (end 33.02 29.21) (width 0.25) (layer F.Cu) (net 14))
 (segment (start 27.94 50.8) (end 33.02 45.72) (width 0.25) (layer F.Cu) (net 14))
 (segment (start 36.83 59.69) (end 36.83 82.55) (width 0.25) (layer B.Cu) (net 14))
 (segment (start 27.94 50.8) (end 36.83 59.69) (width 0.25) (layer B.Cu) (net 14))
 (segment (start 30.48 43.18) (end 30.48 29.21) (width 0.25) (layer F.Cu) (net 15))
 (segment (start 27.94 45.72) (end 30.48 43.18) (width 0.25) (layer F.Cu) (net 15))
 (via (at 50.8 68.58) (size 0.8) (drill 0.4) (layers F.Cu B.Cu) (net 15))
 (segment (start 27.94 45.72) (end 50.8 68.58) (width 0.25) (layer B.Cu) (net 15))
 (segment (start 58.42 76.2) (end 58.42 82.55) (width 0.25) (layer F.Cu) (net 15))
 (segment (start 50.8 68.58) (end 58.42 76.2) (width 0.25) (layer F.Cu) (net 15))
 (segment (start 27.94 40.64) (end 27.94 29.21) (width 0.25) (layer F.Cu) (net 16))
 (via (at 45.72 59.69) (size 0.8) (drill 0.4) (layers F.Cu B.Cu) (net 16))
 (segment (start 27.94 41.91) (end 45.72 59.69) (width 0.25) (layer B.Cu) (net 16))
 (segment (start 27.94 40.64) (end 27.94 41.91) (width 0.25) (layer B.Cu) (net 16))
 (segment (start 46.99 60.96) (end 58.42 60.96) (width 0.25) (layer F.Cu) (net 16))
 (segment (start 45.72 59.69) (end 46.99 60.96) (width 0.25) (layer F.Cu) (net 16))
 (segment (start 105.41 81.28) (end 153.67 81.28) (width 0.25) (layer B.Cu) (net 9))
 (segment (start 157.48 77.47) (end 166.37 77.47) (width 0.25) (layer B.Cu) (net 9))
 (segment (start 153.67 81.28) (end 157.48 77.47) (width 0.25) (layer B.Cu) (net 9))
 (via (at 49.53 41.91) (size 0.8) (drill 0.4) (layers F.Cu B.Cu) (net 9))
 (segment (start 66.04 41.91) (end 49.53 41.91) (width 0.25) (layer F.Cu) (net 9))
 (segment (start 105.41 81.28) (end 66.04 41.91) (width 0.25) (layer F.Cu) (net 9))
 (via (at 46.355 37.555) (size 0.8) (drill 0.4) (layers F.Cu B.Cu) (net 9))
 (segment (start 49.53 40.73) (end 46.355 37.555) (width 0.25) (layer B.Cu) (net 9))
 (segment (start 49.53 41.91) (end 49.53 40.73) (width 0.25) (layer B.Cu) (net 9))
 (via (at 46.550153 32.824847) (size 0.8) (drill 0.4) (layers F.Cu B.Cu) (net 9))
 (segment (start 46.355 33.02) (end 46.550153 32.824847) (width 0.25) (layer F.Cu) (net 9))
 (segment (start 46.355 37.555) (end 46.355 33.02) (width 0.25) (layer F.Cu) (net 9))
 (segment (start 45.72 31.994694) (end 45.72 29.21) (width 0.25) (layer B.Cu) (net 9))
 (segment (start 46.550153 32.824847) (end 45.72 31.994694) (width 0.25) (layer B.Cu) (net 9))
 (segment (start 140.97 91.44) (end 144.78 95.25) (width 0.25) (layer B.Cu) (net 10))
 (segment (start 105.41 91.44) (end 140.97 91.44) (width 0.25) (layer B.Cu) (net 10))
 (via (at 48.26 35.56) (size 0.8) (drill 0.4) (layers F.Cu B.Cu) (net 10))
 (segment (start 43.18 30.48) (end 48.26 35.56) (width 0.25) (layer B.Cu) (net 10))
 (segment (start 43.18 29.21) (end 43.18 30.48) (width 0.25) (layer B.Cu) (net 10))
 (via (at 59.055 39.915) (size 0.8) (drill 0.4) (layers F.Cu B.Cu) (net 10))
 (segment (start 52.615 39.915) (end 59.055 39.915) (width 0.25) (layer F.Cu) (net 10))
 (segment (start 48.26 35.56) (end 52.615 39.915) (width 0.25) (layer F.Cu) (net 10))
 (segment (start 59.055 39.915) (end 60.235 39.915) (width 0.25) (layer B.Cu) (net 10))
 (segment (start 60.235 39.915) (end 94.615 74.295) (width 0.25) (layer B.Cu) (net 10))
 (segment (start 94.615 80.645) (end 105.41 91.44) (width 0.25) (layer B.Cu) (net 10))
 (segment (start 94.615 74.295) (end 94.615 80.645) (width 0.25) (layer B.Cu) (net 10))
 (segment (start 105.41 86.36) (end 169.545 86.36) (width 0.25) (layer B.Cu) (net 8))
 (segment (start 178.435 77.47) (end 188.595 77.47) (width 0.25) (layer B.Cu) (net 8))
 (segment (start 169.545 86.36) (end 178.435 77.47) (width 0.25) (layer B.Cu) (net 8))
 (segment (start 105.41 86.36) (end 95.885 76.835) (width 0.25) (layer B.Cu) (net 8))
 (segment (start 95.885 76.835) (end 95.885 74.295) (width 0.25) (layer B.Cu) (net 8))
 (via (at 59.055 38.735) (size 0.8) (drill 0.4) (layers F.Cu B.Cu) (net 8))
 (segment (start 60.325 38.735) (end 59.055 38.735) (width 0.25) (layer B.Cu) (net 8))
 (segment (start 95.885 74.295) (end 60.325 38.735) (width 0.25) (layer B.Cu) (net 8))
 (segment (start 54.374999 39.134999) (end 48.26 33.02) (width 0.25) (layer F.Cu) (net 8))
 (segment (start 58.655001 39.134999) (end 54.374999 39.134999) (width 0.25) (layer F.Cu) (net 8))
 (via (at 48.26 33.02) (size 0.8) (drill 0.4) (layers F.Cu B.Cu) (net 8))
 (segment (start 59.055 38.735) (end 58.655001 39.134999) (width 0.25) (layer F.Cu) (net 8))
 (segment (start 48.26 33.02) (end 48.26 29.21) (width 0.25) (layer B.Cu) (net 8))
 (segment (start 106.224001 55.065999) (end 192.584001 55.065999) (width 0.25) (layer F.Cu) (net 7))
 (segment (start 105.41 55.88) (end 106.224001 55.065999) (width 0.25) (layer F.Cu) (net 7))
 (segment (start 200.025 47.625) (end 210.185 47.625) (width 0.25) (layer F.Cu) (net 7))
 (segment (start 192.584001 55.065999) (end 200.025 47.625) (width 0.25) (layer F.Cu) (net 7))
 (via (at 69.85 29.21) (size 0.8) (drill 0.4) (layers F.Cu B.Cu) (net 7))
 (segment (start 95.494999 54.854999) (end 69.85 29.21) (width 0.25) (layer B.Cu) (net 7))
 (segment (start 104.384999 54.854999) (end 95.494999 54.854999) (width 0.25) (layer B.Cu) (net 7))
 (segment (start 105.41 55.88) (end 104.384999 54.854999) (width 0.25) (layer B.Cu) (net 7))
 (segment (start 69.85 29.21) (end 67.945 27.305) (width 0.25) (layer F.Cu) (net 7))
 (segment (start 52.705 27.305) (end 50.8 29.21) (width 0.25) (layer F.Cu) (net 7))
 (segment (start 67.945 27.305) (end 52.705 27.305) (width 0.25) (layer F.Cu) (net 7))
 (segment (start 105.41 71.12) (end 118.745 71.12) (width 0.25) (layer B.Cu) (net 6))
 (segment (start 133.35 56.515) (end 144.78 56.515) (width 0.25) (layer B.Cu) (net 6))
 (segment (start 118.745 71.12) (end 133.35 56.515) (width 0.25) (layer B.Cu) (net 6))
 (via (at 58.42 34.29) (size 0.8) (drill 0.4) (layers F.Cu B.Cu) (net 6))
 (segment (start 53.34 29.21) (end 58.42 34.29) (width 0.25) (layer B.Cu) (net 6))
 (via (at 65.405 39.915) (size 0.8) (drill 0.4) (layers F.Cu B.Cu) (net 6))
 (segment (start 64.045 39.915) (end 65.405 39.915) (width 0.25) (layer F.Cu) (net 6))
 (segment (start 58.42 34.29) (end 64.045 39.915) (width 0.25) (layer F.Cu) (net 6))
 (segment (start 74.205 39.915) (end 105.41 71.12) (width 0.25) (layer B.Cu) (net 6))
 (segment (start 65.405 39.915) (end 74.205 39.915) (width 0.25) (layer B.Cu) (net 6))
 (segment (start 105.41 60.96) (end 114.935 60.96) (width 0.25) (layer B.Cu) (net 5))
 (segment (start 137.16 38.735) (end 166.37 38.735) (width 0.25) (layer B.Cu) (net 5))
 (segment (start 114.935 60.96) (end 137.16 38.735) (width 0.25) (layer B.Cu) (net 5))
 (via (at 60.325 33.655) (size 0.8) (drill 0.4) (layers F.Cu B.Cu) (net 5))
 (segment (start 55.88 29.21) (end 60.325 33.655) (width 0.25) (layer B.Cu) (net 5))
 (via (at 74.93 39.37) (size 0.8) (drill 0.4) (layers F.Cu B.Cu) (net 5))
 (segment (start 66.04 39.37) (end 74.93 39.37) (width 0.25) (layer F.Cu) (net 5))
 (segment (start 60.325 33.655) (end 66.04 39.37) (width 0.25) (layer F.Cu) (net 5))
 (segment (start 74.93 39.37) (end 94.615 59.055) (width 0.25) (layer B.Cu) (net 5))
 (segment (start 103.505 59.055) (end 105.41 60.96) (width 0.25) (layer B.Cu) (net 5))
 (segment (start 94.615 59.055) (end 103.505 59.055) (width 0.25) (layer B.Cu) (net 5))
 (segment (start 105.41 66.04) (end 117.475 66.04) (width 0.25) (layer B.Cu) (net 4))
 (segment (start 117.475 66.04) (end 135.255 48.26) (width 0.25) (layer B.Cu) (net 4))
 (segment (start 135.255 48.26) (end 167.005 48.26) (width 0.25) (layer B.Cu) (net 4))
 (segment (start 176.53 38.735) (end 188.595 38.735) (width 0.25) (layer B.Cu) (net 4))
 (segment (start 167.005 48.26) (end 176.53 38.735) (width 0.25) (layer B.Cu) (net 4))
 (via (at 61.399847 32.824847) (size 0.8) (drill 0.4) (layers F.Cu B.Cu) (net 4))
 (segment (start 61.399847 32.189847) (end 61.399847 32.824847) (width 0.25) (layer B.Cu) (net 4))
 (segment (start 58.42 29.21) (end 61.399847 32.189847) (width 0.25) (layer B.Cu) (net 4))
 (segment (start 61.399847 32.824847) (end 67.31 38.735) (width 0.25) (layer F.Cu) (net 4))
 (segment (start 76.744999 38.644999) (end 76.835 38.735) (width 0.25) (layer F.Cu) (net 4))
 (via (at 76.835 38.735) (size 0.8) (drill 0.4) (layers F.Cu B.Cu) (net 4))
 (segment (start 67.400001 38.644999) (end 76.744999 38.644999) (width 0.25) (layer F.Cu) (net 4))
 (segment (start 67.31 38.735) (end 67.400001 38.644999) (width 0.25) (layer F.Cu) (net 4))
 (via (at 93.345 55.155) (size 0.8) (drill 0.4) (layers F.Cu B.Cu) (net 4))
 (segment (start 93.255 55.155) (end 93.345 55.155) (width 0.25) (layer B.Cu) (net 4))
 (segment (start 76.835 38.735) (end 93.255 55.155) (width 0.25) (layer B.Cu) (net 4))
 (segment (start 94.525 55.155) (end 105.41 66.04) (width 0.25) (layer F.Cu) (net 4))
 (segment (start 93.345 55.155) (end 94.525 55.155) (width 0.25) (layer F.Cu) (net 4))
 (segment (start 105.41 76.2) (end 125.73 76.2) (width 0.25) (layer B.Cu) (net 3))
 (segment (start 125.73 76.2) (end 129.54 72.39) (width 0.25) (layer B.Cu) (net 3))
 (segment (start 196.215 72.39) (end 210.185 86.36) (width 0.25) (layer B.Cu) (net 3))
 (segment (start 129.54 72.39) (end 196.215 72.39) (width 0.25) (layer B.Cu) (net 3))
 (segment (start 105.41 76.2) (end 70.485 41.275) (width 0.25) (layer B.Cu) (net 3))
 (via (at 61.595 38.735) (size 0.8) (drill 0.4) (layers F.Cu B.Cu) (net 3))
 (segment (start 64.135 41.275) (end 61.595 38.735) (width 0.25) (layer B.Cu) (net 3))
 (segment (start 70.485 41.275) (end 64.135 41.275) (width 0.25) (layer B.Cu) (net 3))
 (via (at 54.61 32.475) (size 0.8) (drill 0.4) (layers F.Cu B.Cu) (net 3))
 (segment (start 60.87 38.735) (end 54.61 32.475) (width 0.25) (layer F.Cu) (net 3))
 (segment (start 61.595 38.735) (end 60.87 38.735) (width 0.25) (layer F.Cu) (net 3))
 (via (at 53.34 31.025) (size 0.8) (drill 0.4) (layers F.Cu B.Cu) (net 3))
 (segment (start 54.61 32.295) (end 53.34 31.025) (width 0.25) (layer B.Cu) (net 3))
 (segment (start 54.61 32.475) (end 54.61 32.295) (width 0.25) (layer B.Cu) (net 3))
 (segment (start 59.145 31.025) (end 60.96 29.21) (width 0.25) (layer F.Cu) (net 3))
 (segment (start 53.34 31.025) (end 59.145 31.025) (width 0.25) (layer F.Cu) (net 3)))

